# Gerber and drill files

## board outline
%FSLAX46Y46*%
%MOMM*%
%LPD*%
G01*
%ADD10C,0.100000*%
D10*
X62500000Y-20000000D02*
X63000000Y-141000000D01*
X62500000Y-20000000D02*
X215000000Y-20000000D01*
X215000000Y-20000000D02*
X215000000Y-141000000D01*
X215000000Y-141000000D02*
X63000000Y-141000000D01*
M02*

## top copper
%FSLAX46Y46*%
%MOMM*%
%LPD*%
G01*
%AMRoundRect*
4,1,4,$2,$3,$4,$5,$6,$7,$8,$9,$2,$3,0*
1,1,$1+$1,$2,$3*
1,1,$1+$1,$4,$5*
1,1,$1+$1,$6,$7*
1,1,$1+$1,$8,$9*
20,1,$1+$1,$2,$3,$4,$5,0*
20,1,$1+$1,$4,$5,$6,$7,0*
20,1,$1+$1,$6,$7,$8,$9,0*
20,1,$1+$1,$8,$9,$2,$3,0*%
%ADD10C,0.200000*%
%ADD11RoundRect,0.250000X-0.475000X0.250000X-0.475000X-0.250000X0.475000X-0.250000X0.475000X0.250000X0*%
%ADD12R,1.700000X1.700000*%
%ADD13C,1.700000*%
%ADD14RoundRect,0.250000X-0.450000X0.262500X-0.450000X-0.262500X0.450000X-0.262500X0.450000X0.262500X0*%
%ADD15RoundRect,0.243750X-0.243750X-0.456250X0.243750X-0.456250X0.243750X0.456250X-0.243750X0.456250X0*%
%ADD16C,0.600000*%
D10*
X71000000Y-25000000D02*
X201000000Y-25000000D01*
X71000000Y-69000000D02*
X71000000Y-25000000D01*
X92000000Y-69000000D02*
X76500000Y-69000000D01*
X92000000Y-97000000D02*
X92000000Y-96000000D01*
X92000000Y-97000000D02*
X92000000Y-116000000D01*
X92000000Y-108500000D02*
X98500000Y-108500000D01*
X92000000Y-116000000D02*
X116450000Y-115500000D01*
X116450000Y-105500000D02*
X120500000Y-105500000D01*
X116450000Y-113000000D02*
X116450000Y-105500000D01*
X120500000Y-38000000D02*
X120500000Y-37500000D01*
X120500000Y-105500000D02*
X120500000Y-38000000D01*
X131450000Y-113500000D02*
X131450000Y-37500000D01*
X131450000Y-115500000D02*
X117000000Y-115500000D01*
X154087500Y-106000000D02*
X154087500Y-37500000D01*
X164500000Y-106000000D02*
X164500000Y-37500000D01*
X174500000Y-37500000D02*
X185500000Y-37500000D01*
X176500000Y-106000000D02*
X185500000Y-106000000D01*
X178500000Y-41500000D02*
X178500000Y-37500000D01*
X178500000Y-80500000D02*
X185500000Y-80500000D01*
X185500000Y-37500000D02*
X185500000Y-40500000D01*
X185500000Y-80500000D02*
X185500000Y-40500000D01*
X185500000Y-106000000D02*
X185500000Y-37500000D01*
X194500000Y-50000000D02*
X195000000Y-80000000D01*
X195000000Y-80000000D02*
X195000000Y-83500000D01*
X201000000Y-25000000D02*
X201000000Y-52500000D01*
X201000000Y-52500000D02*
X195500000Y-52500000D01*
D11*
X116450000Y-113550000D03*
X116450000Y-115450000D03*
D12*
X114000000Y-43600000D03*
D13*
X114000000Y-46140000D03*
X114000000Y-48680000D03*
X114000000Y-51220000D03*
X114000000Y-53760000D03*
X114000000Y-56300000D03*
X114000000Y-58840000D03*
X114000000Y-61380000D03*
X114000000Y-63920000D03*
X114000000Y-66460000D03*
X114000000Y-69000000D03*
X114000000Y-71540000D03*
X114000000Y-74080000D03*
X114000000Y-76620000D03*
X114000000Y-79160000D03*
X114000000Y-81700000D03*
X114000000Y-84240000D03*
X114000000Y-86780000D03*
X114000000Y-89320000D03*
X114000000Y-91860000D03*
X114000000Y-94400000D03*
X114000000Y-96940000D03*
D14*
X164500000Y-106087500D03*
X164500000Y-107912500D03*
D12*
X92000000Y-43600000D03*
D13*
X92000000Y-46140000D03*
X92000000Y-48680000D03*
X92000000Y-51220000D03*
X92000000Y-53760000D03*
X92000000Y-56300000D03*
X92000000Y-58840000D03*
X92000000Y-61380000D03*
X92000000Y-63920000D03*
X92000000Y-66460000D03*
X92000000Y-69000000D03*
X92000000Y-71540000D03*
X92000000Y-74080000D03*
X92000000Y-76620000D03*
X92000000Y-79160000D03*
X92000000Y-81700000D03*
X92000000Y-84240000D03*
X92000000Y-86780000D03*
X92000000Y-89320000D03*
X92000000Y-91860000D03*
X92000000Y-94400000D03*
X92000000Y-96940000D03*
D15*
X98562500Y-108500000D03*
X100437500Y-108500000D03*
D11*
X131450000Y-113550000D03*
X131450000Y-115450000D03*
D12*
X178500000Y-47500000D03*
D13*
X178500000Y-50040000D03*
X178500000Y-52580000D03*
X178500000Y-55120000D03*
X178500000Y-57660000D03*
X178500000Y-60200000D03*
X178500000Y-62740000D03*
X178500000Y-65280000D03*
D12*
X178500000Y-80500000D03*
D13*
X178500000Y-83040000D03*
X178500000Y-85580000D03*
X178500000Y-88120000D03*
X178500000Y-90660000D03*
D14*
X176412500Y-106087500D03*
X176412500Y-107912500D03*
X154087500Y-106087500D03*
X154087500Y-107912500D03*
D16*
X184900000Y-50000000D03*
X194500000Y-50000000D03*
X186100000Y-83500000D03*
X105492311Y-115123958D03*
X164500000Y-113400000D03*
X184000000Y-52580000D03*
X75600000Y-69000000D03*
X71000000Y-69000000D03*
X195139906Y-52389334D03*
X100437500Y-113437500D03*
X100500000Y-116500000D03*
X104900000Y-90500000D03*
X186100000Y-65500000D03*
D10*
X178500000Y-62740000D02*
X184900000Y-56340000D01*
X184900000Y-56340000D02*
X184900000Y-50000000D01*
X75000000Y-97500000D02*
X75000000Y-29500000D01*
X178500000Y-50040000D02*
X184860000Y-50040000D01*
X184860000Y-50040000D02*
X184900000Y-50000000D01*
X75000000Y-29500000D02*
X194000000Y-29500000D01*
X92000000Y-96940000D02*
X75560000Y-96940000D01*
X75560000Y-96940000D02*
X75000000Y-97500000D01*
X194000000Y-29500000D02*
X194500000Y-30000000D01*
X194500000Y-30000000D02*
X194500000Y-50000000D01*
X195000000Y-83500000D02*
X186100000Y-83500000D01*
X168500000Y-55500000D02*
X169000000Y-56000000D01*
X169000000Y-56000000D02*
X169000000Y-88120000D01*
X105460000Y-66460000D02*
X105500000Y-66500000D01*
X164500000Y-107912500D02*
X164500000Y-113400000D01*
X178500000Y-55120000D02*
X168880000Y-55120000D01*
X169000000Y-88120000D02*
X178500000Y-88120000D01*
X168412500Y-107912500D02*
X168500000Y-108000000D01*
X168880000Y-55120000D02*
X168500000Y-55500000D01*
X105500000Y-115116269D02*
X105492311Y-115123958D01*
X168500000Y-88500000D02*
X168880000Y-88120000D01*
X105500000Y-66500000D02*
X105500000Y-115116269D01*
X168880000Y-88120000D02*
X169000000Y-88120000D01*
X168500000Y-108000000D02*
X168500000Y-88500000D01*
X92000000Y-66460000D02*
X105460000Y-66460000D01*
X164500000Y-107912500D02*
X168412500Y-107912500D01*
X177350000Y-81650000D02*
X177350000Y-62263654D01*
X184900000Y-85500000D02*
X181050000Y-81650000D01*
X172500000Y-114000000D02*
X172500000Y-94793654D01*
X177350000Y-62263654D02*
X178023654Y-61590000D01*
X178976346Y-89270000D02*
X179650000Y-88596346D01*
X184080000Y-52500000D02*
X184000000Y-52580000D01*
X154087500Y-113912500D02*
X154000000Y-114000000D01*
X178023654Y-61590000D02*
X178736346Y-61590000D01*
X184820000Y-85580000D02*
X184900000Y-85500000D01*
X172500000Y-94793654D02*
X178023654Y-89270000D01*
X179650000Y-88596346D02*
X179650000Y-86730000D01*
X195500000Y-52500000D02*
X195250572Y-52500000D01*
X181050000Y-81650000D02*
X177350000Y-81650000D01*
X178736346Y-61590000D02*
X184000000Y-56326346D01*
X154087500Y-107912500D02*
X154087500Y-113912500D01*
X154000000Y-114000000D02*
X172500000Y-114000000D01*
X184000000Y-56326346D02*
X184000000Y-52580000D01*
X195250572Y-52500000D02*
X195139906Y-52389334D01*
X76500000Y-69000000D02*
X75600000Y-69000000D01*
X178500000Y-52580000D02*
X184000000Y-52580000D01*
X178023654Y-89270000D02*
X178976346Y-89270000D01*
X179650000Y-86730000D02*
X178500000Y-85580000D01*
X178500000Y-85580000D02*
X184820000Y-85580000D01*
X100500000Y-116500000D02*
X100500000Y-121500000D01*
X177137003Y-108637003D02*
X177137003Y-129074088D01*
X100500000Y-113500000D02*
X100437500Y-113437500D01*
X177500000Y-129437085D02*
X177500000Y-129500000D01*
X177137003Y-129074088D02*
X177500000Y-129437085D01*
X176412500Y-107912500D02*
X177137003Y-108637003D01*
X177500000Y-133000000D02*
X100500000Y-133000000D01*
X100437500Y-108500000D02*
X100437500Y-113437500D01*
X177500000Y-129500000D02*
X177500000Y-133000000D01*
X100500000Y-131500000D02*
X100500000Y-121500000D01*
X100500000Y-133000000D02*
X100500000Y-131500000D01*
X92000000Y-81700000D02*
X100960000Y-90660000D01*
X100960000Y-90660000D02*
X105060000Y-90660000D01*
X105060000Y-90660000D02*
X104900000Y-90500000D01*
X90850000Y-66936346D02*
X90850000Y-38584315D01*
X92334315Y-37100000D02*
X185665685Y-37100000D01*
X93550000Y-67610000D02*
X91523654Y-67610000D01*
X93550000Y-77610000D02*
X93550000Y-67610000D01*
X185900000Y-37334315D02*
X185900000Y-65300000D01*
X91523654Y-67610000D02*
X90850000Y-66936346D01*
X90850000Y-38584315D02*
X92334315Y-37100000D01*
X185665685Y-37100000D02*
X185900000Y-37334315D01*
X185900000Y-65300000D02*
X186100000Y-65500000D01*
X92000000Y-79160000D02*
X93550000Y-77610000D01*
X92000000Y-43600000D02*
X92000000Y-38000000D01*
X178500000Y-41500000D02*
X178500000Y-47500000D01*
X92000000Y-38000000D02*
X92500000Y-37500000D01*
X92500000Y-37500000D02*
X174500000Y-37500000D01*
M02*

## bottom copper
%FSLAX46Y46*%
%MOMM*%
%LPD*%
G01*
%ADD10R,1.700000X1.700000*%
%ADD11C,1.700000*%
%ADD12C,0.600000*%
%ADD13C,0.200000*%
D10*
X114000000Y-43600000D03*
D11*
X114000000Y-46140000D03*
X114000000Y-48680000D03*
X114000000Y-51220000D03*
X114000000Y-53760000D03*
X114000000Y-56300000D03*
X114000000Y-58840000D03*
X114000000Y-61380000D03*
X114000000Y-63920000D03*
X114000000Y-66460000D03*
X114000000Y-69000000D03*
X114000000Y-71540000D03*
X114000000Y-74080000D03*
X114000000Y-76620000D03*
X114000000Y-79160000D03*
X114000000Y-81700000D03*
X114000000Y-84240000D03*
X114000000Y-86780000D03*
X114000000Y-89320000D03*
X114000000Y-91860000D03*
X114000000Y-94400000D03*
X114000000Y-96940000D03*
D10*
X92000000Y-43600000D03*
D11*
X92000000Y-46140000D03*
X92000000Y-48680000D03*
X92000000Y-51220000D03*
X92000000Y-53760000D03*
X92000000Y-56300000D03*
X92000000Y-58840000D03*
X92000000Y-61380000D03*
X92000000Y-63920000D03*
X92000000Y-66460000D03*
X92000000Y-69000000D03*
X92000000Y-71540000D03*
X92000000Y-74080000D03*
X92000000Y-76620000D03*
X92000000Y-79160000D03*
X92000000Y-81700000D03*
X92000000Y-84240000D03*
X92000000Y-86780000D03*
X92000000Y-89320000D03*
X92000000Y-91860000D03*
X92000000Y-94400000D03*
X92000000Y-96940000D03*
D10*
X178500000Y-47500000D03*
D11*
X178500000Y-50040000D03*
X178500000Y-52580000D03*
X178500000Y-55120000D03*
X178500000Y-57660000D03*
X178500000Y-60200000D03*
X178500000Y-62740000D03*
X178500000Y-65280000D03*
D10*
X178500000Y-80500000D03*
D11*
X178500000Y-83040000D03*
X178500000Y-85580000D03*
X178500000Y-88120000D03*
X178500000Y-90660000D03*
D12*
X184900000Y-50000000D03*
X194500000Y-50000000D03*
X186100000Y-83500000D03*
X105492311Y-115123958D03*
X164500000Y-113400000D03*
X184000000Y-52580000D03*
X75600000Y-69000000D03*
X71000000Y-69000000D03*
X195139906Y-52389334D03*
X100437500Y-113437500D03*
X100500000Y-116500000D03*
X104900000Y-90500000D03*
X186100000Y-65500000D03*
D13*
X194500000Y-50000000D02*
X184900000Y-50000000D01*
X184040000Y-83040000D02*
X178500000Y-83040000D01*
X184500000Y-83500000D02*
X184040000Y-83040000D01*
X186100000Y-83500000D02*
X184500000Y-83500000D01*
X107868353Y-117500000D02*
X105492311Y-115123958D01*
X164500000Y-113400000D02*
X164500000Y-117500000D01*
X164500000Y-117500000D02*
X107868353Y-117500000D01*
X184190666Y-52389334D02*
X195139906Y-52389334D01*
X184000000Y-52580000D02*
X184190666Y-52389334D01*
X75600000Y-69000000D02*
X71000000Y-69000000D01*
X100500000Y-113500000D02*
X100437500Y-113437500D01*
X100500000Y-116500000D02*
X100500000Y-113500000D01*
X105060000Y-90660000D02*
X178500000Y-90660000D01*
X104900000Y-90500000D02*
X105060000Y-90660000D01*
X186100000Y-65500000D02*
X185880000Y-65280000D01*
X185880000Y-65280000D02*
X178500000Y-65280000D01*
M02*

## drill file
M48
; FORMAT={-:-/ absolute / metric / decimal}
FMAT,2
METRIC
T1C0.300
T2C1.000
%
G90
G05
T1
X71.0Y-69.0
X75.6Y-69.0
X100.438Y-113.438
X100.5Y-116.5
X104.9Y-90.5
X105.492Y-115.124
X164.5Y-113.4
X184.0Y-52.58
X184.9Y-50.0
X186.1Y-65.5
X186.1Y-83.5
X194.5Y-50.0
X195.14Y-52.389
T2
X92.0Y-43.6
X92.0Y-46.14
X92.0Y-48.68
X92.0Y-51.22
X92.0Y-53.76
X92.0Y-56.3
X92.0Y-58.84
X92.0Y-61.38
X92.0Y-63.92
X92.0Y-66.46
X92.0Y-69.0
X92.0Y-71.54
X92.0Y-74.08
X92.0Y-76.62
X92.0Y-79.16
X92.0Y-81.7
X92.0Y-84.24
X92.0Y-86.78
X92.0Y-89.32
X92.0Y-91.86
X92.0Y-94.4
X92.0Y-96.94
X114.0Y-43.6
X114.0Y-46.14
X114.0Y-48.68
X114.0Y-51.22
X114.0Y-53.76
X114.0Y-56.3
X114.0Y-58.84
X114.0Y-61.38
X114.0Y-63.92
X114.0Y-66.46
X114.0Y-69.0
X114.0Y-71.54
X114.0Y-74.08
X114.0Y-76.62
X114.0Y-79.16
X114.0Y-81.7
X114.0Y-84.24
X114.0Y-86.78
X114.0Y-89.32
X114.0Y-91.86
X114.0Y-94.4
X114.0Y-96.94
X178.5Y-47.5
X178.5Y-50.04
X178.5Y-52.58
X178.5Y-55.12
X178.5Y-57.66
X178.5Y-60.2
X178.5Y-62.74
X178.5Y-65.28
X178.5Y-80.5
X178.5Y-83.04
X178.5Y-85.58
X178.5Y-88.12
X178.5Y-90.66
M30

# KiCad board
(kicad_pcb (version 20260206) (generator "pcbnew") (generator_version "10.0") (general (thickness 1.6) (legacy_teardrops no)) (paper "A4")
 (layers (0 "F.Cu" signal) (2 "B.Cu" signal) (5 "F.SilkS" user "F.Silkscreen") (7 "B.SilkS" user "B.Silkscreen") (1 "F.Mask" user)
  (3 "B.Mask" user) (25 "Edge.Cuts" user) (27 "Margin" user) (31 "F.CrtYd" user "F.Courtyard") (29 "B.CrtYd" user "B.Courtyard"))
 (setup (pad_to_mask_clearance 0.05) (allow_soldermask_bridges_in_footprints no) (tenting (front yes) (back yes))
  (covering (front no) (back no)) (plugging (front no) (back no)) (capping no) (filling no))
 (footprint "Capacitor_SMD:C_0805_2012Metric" (layer "F.Cu") (at 116.45 114.5 -90)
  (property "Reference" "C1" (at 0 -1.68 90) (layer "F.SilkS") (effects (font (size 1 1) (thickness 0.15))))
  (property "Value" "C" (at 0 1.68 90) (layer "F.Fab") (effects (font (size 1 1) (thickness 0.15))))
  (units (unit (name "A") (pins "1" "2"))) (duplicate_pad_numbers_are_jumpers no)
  (pad "1" smd roundrect (at -0.95 0 270) (size 1 1.45) (layers "F.Cu" "F.Mask" "F.Paste") (roundrect_rratio 0.25) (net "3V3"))
  (pad "2" smd roundrect (at 0.95 0 270) (size 1 1.45) (layers "F.Cu" "F.Mask" "F.Paste") (roundrect_rratio 0.25) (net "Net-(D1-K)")))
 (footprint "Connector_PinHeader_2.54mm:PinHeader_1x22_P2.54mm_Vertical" (layer "F.Cu") (at 114 43.6)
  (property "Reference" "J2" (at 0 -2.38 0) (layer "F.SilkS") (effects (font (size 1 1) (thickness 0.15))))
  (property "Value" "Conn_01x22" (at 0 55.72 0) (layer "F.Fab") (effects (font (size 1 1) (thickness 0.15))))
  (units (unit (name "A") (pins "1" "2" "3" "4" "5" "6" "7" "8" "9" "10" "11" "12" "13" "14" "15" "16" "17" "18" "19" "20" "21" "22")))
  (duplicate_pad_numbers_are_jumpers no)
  (pad "1" thru_hole rect (at 0 0) (size 1.7 1.7) (drill 1) (layers "*.Cu" "*.Mask") (remove_unused_layers no)
   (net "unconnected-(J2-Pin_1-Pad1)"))
  (pad "2" thru_hole circle (at 0 2.54) (size 1.7 1.7) (drill 1) (layers "*.Cu" "*.Mask") (remove_unused_layers no)
   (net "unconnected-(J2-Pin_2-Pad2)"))
  (pad "3" thru_hole circle (at 0 5.08) (size 1.7 1.7) (drill 1) (layers "*.Cu" "*.Mask") (remove_unused_layers no)
   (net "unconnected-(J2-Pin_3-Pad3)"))
  (pad "4" thru_hole circle (at 0 7.62) (size 1.7 1.7) (drill 1) (layers "*.Cu" "*.Mask") (remove_unused_layers no)
   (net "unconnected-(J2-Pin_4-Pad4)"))
  (pad "5" thru_hole circle (at 0 10.16) (size 1.7 1.7) (drill 1) (layers "*.Cu" "*.Mask") (remove_unused_layers no)
   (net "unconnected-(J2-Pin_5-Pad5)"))
  (pad "6" thru_hole circle (at 0 12.7) (size 1.7 1.7) (drill 1) (layers "*.Cu" "*.Mask") (remove_unused_layers no)
   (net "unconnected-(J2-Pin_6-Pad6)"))
  (pad "7" thru_hole circle (at 0 15.24) (size 1.7 1.7) (drill 1) (layers "*.Cu" "*.Mask") (remove_unused_layers no)
   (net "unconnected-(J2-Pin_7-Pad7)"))
  (pad "8" thru_hole circle (at 0 17.78) (size 1.7 1.7) (drill 1) (layers "*.Cu" "*.Mask") (remove_unused_layers no)
   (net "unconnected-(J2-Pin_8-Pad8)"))
  (pad "9" thru_hole circle (at 0 20.32) (size 1.7 1.7) (drill 1) (layers "*.Cu" "*.Mask") (remove_unused_layers no)
   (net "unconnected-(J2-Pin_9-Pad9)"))
  (pad "10" thru_hole circle (at 0 22.86) (size 1.7 1.7) (drill 1) (layers "*.Cu" "*.Mask") (remove_unused_layers no)
   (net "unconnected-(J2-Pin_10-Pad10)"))
  (pad "11" thru_hole circle (at 0 25.4) (size 1.7 1.7) (drill 1) (layers "*.Cu" "*.Mask") (remove_unused_layers no)
   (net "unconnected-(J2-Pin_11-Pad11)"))
  (pad "12" thru_hole circle (at 0 27.94) (size 1.7 1.7) (drill 1) (layers "*.Cu" "*.Mask") (remove_unused_layers no)
   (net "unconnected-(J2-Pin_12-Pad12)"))
  (pad "13" thru_hole circle (at 0 30.48) (size 1.7 1.7) (drill 1) (layers "*.Cu" "*.Mask") (remove_unused_layers no)
   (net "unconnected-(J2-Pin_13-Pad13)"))
  (pad "14" thru_hole circle (at 0 33.02) (size 1.7 1.7) (drill 1) (layers "*.Cu" "*.Mask") (remove_unused_layers no)
   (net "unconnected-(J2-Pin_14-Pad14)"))
  (pad "15" thru_hole circle (at 0 35.56) (size 1.7 1.7) (drill 1) (layers "*.Cu" "*.Mask") (remove_unused_layers no)
   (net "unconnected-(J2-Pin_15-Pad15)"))
  (pad "16" thru_hole circle (at 0 38.1) (size 1.7 1.7) (drill 1) (layers "*.Cu" "*.Mask") (remove_unused_layers no)
   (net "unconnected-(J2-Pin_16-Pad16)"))
  (pad "17" thru_hole circle (at 0 40.64) (size 1.7 1.7) (drill 1) (layers "*.Cu" "*.Mask") (remove_unused_layers no)
   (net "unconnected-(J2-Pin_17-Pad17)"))
  (pad "18" thru_hole circle (at 0 43.18) (size 1.7 1.7) (drill 1) (layers "*.Cu" "*.Mask") (remove_unused_layers no)
   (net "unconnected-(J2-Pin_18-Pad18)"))
  (pad "19" thru_hole circle (at 0 45.72) (size 1.7 1.7) (drill 1) (layers "*.Cu" "*.Mask") (remove_unused_layers no)
   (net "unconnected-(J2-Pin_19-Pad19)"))
  (pad "20" thru_hole circle (at 0 48.26) (size 1.7 1.7) (drill 1) (layers "*.Cu" "*.Mask") (remove_unused_layers no)
   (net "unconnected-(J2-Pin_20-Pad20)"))
  (pad "21" thru_hole circle (at 0 50.8) (size 1.7 1.7) (drill 1) (layers "*.Cu" "*.Mask") (remove_unused_layers no)
   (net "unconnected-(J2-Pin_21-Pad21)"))
  (pad "22" thru_hole circle (at 0 53.34) (size 1.7 1.7) (drill 1) (layers "*.Cu" "*.Mask") (remove_unused_layers no)
   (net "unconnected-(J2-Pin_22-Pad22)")))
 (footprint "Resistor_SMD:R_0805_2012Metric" (layer "F.Cu") (at 164.5 107 -90)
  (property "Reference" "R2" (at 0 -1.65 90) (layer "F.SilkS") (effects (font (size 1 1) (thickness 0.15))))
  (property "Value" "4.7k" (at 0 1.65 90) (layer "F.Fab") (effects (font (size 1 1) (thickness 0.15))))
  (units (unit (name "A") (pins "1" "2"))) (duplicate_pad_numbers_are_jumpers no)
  (pad "1" smd roundrect (at -0.9125 0 270) (size 1.025 1.4) (layers "F.Cu" "F.Mask" "F.Paste") (roundrect_rratio 0.243902) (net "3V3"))
  (pad "2" smd roundrect (at 0.9125 0 270) (size 1.025 1.4) (layers "F.Cu" "F.Mask" "F.Paste") (roundrect_rratio 0.243902)
   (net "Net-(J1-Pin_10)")))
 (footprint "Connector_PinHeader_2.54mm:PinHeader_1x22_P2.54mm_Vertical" (layer "F.Cu") (at 92 43.6)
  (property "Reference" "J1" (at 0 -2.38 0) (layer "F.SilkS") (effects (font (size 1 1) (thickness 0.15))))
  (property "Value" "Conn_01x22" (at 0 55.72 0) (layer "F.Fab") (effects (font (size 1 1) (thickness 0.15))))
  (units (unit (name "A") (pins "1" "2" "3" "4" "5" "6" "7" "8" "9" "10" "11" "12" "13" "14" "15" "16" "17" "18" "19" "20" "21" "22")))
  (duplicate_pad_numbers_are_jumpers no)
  (pad "1" thru_hole rect (at 0 0) (size 1.7 1.7) (drill 1) (layers "*.Cu" "*.Mask") (remove_unused_layers no) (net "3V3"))
  (pad "2" thru_hole circle (at 0 2.54) (size 1.7 1.7) (drill 1) (layers "*.Cu" "*.Mask") (remove_unused_layers no)
   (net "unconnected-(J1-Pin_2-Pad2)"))
  (pad "3" thru_hole circle (at 0 5.08) (size 1.7 1.7) (drill 1) (layers "*.Cu" "*.Mask") (remove_unused_layers no)
   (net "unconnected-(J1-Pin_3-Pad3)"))
  (pad "4" thru_hole circle (at 0 7.62) (size 1.7 1.7) (drill 1) (layers "*.Cu" "*.Mask") (remove_unused_layers no)
   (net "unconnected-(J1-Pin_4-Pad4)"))
  (pad "5" thru_hole circle (at 0 10.16) (size 1.7 1.7) (drill 1) (layers "*.Cu" "*.Mask") (remove_unused_layers no)
   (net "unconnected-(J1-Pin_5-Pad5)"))
  (pad "6" thru_hole circle (at 0 12.7) (size 1.7 1.7) (drill 1) (layers "*.Cu" "*.Mask") (remove_unused_layers no)
   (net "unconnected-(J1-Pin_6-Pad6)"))
  (pad "7" thru_hole circle (at 0 15.24) (size 1.7 1.7) (drill 1) (layers "*.Cu" "*.Mask") (remove_unused_layers no)
   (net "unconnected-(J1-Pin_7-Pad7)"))
  (pad "8" thru_hole circle (at 0 17.78) (size 1.7 1.7) (drill 1) (layers "*.Cu" "*.Mask") (remove_unused_layers no)
   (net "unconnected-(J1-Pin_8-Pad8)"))
  (pad "9" thru_hole circle (at 0 20.32) (size 1.7 1.7) (drill 1) (layers "*.Cu" "*.Mask") (remove_unused_layers no)
   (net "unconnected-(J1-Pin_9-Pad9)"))
  (pad "10" thru_hole circle (at 0 22.86) (size 1.7 1.7) (drill 1) (layers "*.Cu" "*.Mask") (remove_unused_layers no)
   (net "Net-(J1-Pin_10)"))
  (pad "11" thru_hole circle (at 0 25.4) (size 1.7 1.7) (drill 1) (layers "*.Cu" "*.Mask") (remove_unused_layers no) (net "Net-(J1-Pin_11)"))
  (pad "12" thru_hole circle (at 0 27.94) (size 1.7 1.7) (drill 1) (layers "*.Cu" "*.Mask") (remove_unused_layers no)
   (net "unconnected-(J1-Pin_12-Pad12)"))
  (pad "13" thru_hole circle (at 0 30.48) (size 1.7 1.7) (drill 1) (layers "*.Cu" "*.Mask") (remove_unused_layers no)
   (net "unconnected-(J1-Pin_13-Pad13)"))
  (pad "14" thru_hole circle (at 0 33.02) (size 1.7 1.7) (drill 1) (layers "*.Cu" "*.Mask") (remove_unused_layers no)
   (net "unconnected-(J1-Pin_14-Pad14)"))
  (pad "15" thru_hole circle (at 0 35.56) (size 1.7 1.7) (drill 1) (layers "*.Cu" "*.Mask") (remove_unused_layers no) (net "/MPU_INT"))
  (pad "16" thru_hole circle (at 0 38.1) (size 1.7 1.7) (drill 1) (layers "*.Cu" "*.Mask") (remove_unused_layers no) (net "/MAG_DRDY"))
  (pad "17" thru_hole circle (at 0 40.64) (size 1.7 1.7) (drill 1) (layers "*.Cu" "*.Mask") (remove_unused_layers no)
   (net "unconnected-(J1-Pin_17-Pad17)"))
  (pad "18" thru_hole circle (at 0 43.18) (size 1.7 1.7) (drill 1) (layers "*.Cu" "*.Mask") (remove_unused_layers no)
   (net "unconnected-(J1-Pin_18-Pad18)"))
  (pad "19" thru_hole circle (at 0 45.72) (size 1.7 1.7) (drill 1) (layers "*.Cu" "*.Mask") (remove_unused_layers no)
   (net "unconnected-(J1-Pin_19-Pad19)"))
  (pad "20" thru_hole circle (at 0 48.26) (size 1.7 1.7) (drill 1) (layers "*.Cu" "*.Mask") (remove_unused_layers no)
   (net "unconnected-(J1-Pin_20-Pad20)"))
  (pad "21" thru_hole circle (at 0 50.8) (size 1.7 1.7) (drill 1) (layers "*.Cu" "*.Mask") (remove_unused_layers no)
   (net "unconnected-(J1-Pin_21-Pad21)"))
  (pad "22" thru_hole circle (at 0 53.34) (size 1.7 1.7) (drill 1) (layers "*.Cu" "*.Mask") (remove_unused_layers no) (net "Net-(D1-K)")))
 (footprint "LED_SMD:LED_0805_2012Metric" (layer "F.Cu") (at 99.5 108.5)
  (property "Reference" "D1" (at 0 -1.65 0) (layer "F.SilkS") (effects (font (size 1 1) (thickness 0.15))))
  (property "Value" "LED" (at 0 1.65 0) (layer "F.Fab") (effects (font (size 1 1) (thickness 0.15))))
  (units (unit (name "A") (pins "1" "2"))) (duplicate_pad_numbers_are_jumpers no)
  (pad "1" smd roundrect (at -0.9375 0) (size 0.975 1.4) (layers "F.Cu" "F.Mask" "F.Paste") (roundrect_rratio 0.25) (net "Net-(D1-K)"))
  (pad "2" smd roundrect (at 0.9375 0) (size 0.975 1.4) (layers "F.Cu" "F.Mask" "F.Paste") (roundrect_rratio 0.25) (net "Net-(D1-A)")))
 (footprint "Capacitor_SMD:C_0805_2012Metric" (layer "F.Cu") (at 131.45 114.5 -90)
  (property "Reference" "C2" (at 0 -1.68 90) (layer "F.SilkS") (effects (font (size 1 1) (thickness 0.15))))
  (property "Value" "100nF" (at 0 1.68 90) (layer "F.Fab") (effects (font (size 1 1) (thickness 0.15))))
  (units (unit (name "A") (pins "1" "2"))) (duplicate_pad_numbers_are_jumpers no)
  (pad "1" smd roundrect (at -0.95 0 270) (size 1 1.45) (layers "F.Cu" "F.Mask" "F.Paste") (roundrect_rratio 0.25) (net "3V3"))
  (pad "2" smd roundrect (at 0.95 0 270) (size 1 1.45) (layers "F.Cu" "F.Mask" "F.Paste") (roundrect_rratio 0.25) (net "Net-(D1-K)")))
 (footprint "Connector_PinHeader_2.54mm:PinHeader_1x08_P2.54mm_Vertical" (layer "F.Cu") (at 178.5 47.5)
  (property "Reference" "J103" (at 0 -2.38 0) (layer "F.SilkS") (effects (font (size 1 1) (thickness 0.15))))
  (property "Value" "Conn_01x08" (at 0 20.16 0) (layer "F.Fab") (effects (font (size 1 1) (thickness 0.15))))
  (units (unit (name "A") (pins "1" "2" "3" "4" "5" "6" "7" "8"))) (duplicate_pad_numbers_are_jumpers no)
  (pad "1" thru_hole rect (at 0 0) (size 1.7 1.7) (drill 1) (layers "*.Cu" "*.Mask") (remove_unused_layers no) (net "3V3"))
  (pad "2" thru_hole circle (at 0 2.54) (size 1.7 1.7) (drill 1) (layers "*.Cu" "*.Mask") (remove_unused_layers no) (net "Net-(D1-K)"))
  (pad "3" thru_hole circle (at 0 5.08) (size 1.7 1.7) (drill 1) (layers "*.Cu" "*.Mask") (remove_unused_layers no) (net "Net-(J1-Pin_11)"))
  (pad "4" thru_hole circle (at 0 7.62) (size 1.7 1.7) (drill 1) (layers "*.Cu" "*.Mask") (remove_unused_layers no) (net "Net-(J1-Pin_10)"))
  (pad "5" thru_hole circle (at 0 10.16) (size 1.7 1.7) (drill 1) (layers "*.Cu" "*.Mask") (remove_unused_layers no)
   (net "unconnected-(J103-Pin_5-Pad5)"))
  (pad "6" thru_hole circle (at 0 12.7) (size 1.7 1.7) (drill 1) (layers "*.Cu" "*.Mask") (remove_unused_layers no)
   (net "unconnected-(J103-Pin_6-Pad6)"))
  (pad "7" thru_hole circle (at 0 15.24) (size 1.7 1.7) (drill 1) (layers "*.Cu" "*.Mask") (remove_unused_layers no) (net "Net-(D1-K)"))
  (pad "8" thru_hole circle (at 0 17.78) (size 1.7 1.7) (drill 1) (layers "*.Cu" "*.Mask") (remove_unused_layers no) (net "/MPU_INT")))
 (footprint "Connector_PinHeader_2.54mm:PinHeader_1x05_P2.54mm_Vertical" (layer "F.Cu") (at 178.5 80.5)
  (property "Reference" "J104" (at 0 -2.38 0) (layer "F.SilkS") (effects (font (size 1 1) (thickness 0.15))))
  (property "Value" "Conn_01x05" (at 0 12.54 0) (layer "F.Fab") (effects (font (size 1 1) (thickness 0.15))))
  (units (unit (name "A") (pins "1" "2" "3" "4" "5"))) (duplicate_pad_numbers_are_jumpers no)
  (pad "1" thru_hole rect (at 0 0) (size 1.7 1.7) (drill 1) (layers "*.Cu" "*.Mask") (remove_unused_layers no) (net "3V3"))
  (pad "2" thru_hole circle (at 0 2.54) (size 1.7 1.7) (drill 1) (layers "*.Cu" "*.Mask") (remove_unused_layers no) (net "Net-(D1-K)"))
  (pad "3" thru_hole circle (at 0 5.08) (size 1.7 1.7) (drill 1) (layers "*.Cu" "*.Mask") (remove_unused_layers no) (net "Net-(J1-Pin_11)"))
  (pad "4" thru_hole circle (at 0 7.62) (size 1.7 1.7) (drill 1) (layers "*.Cu" "*.Mask") (remove_unused_layers no) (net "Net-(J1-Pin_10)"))
  (pad "5" thru_hole circle (at 0 10.16) (size 1.7 1.7) (drill 1) (layers "*.Cu" "*.Mask") (remove_unused_layers no) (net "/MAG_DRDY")))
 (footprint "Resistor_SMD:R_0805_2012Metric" (layer "F.Cu") (at 176.4125 107 -90)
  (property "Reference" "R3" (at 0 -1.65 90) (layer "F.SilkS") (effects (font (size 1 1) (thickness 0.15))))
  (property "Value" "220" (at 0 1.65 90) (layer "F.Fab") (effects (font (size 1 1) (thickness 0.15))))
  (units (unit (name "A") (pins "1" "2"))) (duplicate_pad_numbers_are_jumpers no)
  (pad "1" smd roundrect (at -0.9125 0 270) (size 1.025 1.4) (layers "F.Cu" "F.Mask" "F.Paste") (roundrect_rratio 0.243902) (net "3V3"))
  (pad "2" smd roundrect (at 0.9125 0 270) (size 1.025 1.4) (layers "F.Cu" "F.Mask" "F.Paste") (roundrect_rratio 0.243902)
   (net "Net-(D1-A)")))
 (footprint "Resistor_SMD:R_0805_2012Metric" (layer "F.Cu") (at 154.0875 107 -90)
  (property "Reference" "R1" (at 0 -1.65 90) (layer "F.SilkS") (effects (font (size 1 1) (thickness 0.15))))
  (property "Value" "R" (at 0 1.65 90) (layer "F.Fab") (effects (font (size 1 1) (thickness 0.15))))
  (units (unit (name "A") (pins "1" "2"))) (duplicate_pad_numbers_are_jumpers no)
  (pad "1" smd roundrect (at -0.9125 0 270) (size 1.025 1.4) (layers "F.Cu" "F.Mask" "F.Paste") (roundrect_rratio 0.243902) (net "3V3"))
  (pad "2" smd roundrect (at 0.9125 0 270) (size 1.025 1.4) (layers "F.Cu" "F.Mask" "F.Paste") (roundrect_rratio 0.243902)
   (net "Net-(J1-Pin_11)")))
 (gr_line (start 71 25) (end 201 25) (stroke (width 0.2) (type default)) (layer "F.Cu") (net "Net-(J1-Pin_11)"))
 (gr_line (start 71 69) (end 71 25) (stroke (width 0.2) (type default)) (layer "F.Cu") (net "Net-(J1-Pin_11)"))
 (gr_line (start 92 69) (end 76.5 69) (stroke (width 0.2) (type default)) (layer "F.Cu") (net "Net-(J1-Pin_11)"))
 (gr_line (start 92 97) (end 92 96) (stroke (width 0.2) (type default)) (layer "F.Cu") (net "Net-(D1-K)"))
 (gr_line (start 92 97) (end 92 116) (stroke (width 0.2) (type default)) (layer "F.Cu") (net "Net-(D1-K)"))
 (gr_line (start 92 108.5) (end 98.5 108.5) (stroke (width 0.2) (type default)) (layer "F.Cu") (net "Net-(D1-K)"))
 (gr_line (start 92 116) (end 116.45 115.5) (stroke (width 0.2) (type default)) (layer "F.Cu") (net "Net-(D1-K)"))
 (gr_line (start 116.45 105.5) (end 120.5 105.5) (stroke (width 0.2) (type default)) (layer "F.Cu") (net "3V3"))
 (gr_line (start 116.45 113) (end 116.45 105.5) (stroke (width 0.2) (type default)) (layer "F.Cu") (net "3V3"))
 (gr_line (start 120.5 38) (end 120.5 37.5) (stroke (width 0.2) (type default)) (layer "F.Cu") (net "3V3"))
 (gr_line (start 120.5 105.5) (end 120.5 38) (stroke (width 0.2) (type default)) (layer "F.Cu") (net "3V3"))
 (gr_line (start 131.45 113.5) (end 131.45 37.5) (stroke (width 0.2) (type default)) (layer "F.Cu") (net "3V3"))
 (gr_line (start 131.45 115.5) (end 117 115.5) (stroke (width 0.2) (type default)) (layer "F.Cu") (net "Net-(D1-K)"))
 (gr_line (start 154.0875 106) (end 154.0875 37.5) (stroke (width 0.2) (type default)) (layer "F.Cu") (net "3V3"))
 (gr_line (start 164.5 106) (end 164.5 37.5) (stroke (width 0.2) (type default)) (layer "F.Cu") (net "3V3"))
 (gr_line (start 174.5 37.5) (end 185.5 37.5) (stroke (width 0.2) (type default)) (layer "F.Cu") (net "3V3"))
 (gr_line (start 176.5 106) (end 185.5 106) (stroke (width 0.2) (type default)) (layer "F.Cu") (net "3V3"))
 (gr_line (start 178.5 41.5) (end 178.5 37.5) (stroke (width 0.2) (type default)) (layer "F.Cu") (net "3V3"))
 (gr_line (start 178.5 80.5) (end 185.5 80.5) (stroke (width 0.2) (type default)) (layer "F.Cu") (net "3V3"))
 (gr_line (start 185.5 37.5) (end 185.5 40.5) (stroke (width 0.2) (type default)) (layer "F.Cu") (net "3V3"))
 (gr_line (start 185.5 80.5) (end 185.5 40.5) (stroke (width 0.2) (type default)) (layer "F.Cu") (net "3V3"))
 (gr_line (start 185.5 106) (end 185.5 37.5) (stroke (width 0.2) (type default)) (layer "F.Cu") (net "3V3"))
 (gr_line (start 194.5 50) (end 195 80) (stroke (width 0.2) (type default)) (layer "F.Cu") (net "Net-(D1-K)"))
 (gr_line (start 195 80) (end 195 83.5) (stroke (width 0.2) (type default)) (layer "F.Cu") (net "Net-(D1-K)"))
 (gr_line (start 201 25) (end 201 52.5) (stroke (width 0.2) (type default)) (layer "F.Cu") (net "Net-(J1-Pin_11)"))
 (gr_line (start 201 52.5) (end 195.5 52.5) (stroke (width 0.2) (type default)) (layer "F.Cu") (net "Net-(J1-Pin_11)"))
 (gr_line (start 62.5 20) (end 63 141) (stroke (width 0.1) (type default)) (layer "Edge.Cuts"))
 (gr_line (start 62.5 20) (end 215 20) (stroke (width 0.1) (type default)) (layer "Edge.Cuts"))
 (gr_line (start 215 20) (end 215 141) (stroke (width 0.1) (type default)) (layer "Edge.Cuts"))
 (gr_line (start 215 141) (end 63 141) (stroke (width 0.1) (type default)) (layer "Edge.Cuts"))
 (segment (start 178.5 62.74) (end 184.9 56.34) (width 0.2) (layer "F.Cu") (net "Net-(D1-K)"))
 (segment (start 184.9 56.34) (end 184.9 50) (width 0.2) (layer "F.Cu") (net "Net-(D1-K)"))
 (segment (start 75 97.5) (end 75 29.5) (width 0.2) (layer "F.Cu") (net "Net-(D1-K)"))
 (segment (start 178.5 50.04) (end 184.86 50.04) (width 0.2) (layer "F.Cu") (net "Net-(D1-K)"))
 (segment (start 184.86 50.04) (end 184.9 50) (width 0.2) (layer "F.Cu") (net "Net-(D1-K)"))
 (segment (start 75 29.5) (end 194 29.5) (width 0.2) (layer "F.Cu") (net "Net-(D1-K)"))
 (segment (start 92 96.94) (end 75.56 96.94) (width 0.2) (layer "F.Cu") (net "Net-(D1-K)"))
 (segment (start 75.56 96.94) (end 75 97.5) (width 0.2) (layer "F.Cu") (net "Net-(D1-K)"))
 (segment (start 194 29.5) (end 194.5 30) (width 0.2) (layer "F.Cu") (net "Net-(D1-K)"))
 (segment (start 194.5 30) (end 194.5 50) (width 0.2) (layer "F.Cu") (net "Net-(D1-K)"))
 (segment (start 195 83.5) (end 186.1 83.5) (width 0.2) (layer "F.Cu") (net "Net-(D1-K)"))
 (via (at 184.9 50) (size 0.6) (drill 0.3) (layers "F.Cu" "B.Cu") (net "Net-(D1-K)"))
 (via (at 194.5 50) (size 0.6) (drill 0.3) (layers "F.Cu" "B.Cu") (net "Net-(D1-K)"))
 (via (at 186.1 83.5) (size 0.6) (drill 0.3) (layers "F.Cu" "B.Cu") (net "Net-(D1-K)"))
 (segment (start 194.5 50) (end 184.9 50) (width 0.2) (layer "B.Cu") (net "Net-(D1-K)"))
 (segment (start 184.04 83.04) (end 178.5 83.04) (width 0.2) (layer "B.Cu") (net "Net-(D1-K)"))
 (segment (start 184.5 83.5) (end 184.04 83.04) (width 0.2) (layer "B.Cu") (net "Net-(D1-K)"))
 (segment (start 186.1 83.5) (end 184.5 83.5) (width 0.2) (layer "B.Cu") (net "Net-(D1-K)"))
 (segment (start 168.5 55.5) (end 169 56) (width 0.2) (layer "F.Cu") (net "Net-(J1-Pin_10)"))
 (segment (start 169 56) (end 169 88.12) (width 0.2) (layer "F.Cu") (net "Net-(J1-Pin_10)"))
 (segment (start 105.46 66.46) (end 105.5 66.5) (width 0.2) (layer "F.Cu") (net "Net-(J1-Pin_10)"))
 (segment (start 164.5 107.9125) (end 164.5 113.4) (width 0.2) (layer "F.Cu") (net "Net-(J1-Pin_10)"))
 (segment (start 178.5 55.12) (end 168.88 55.12) (width 0.2) (layer "F.Cu") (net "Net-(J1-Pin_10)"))
 (segment (start 169 88.12) (end 178.5 88.12) (width 0.2) (layer "F.Cu") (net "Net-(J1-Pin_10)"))
 (segment (start 168.4125 107.9125) (end 168.5 108) (width 0.2) (layer "F.Cu") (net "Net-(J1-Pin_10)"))
 (segment (start 168.88 55.12) (end 168.5 55.5) (width 0.2) (layer "F.Cu") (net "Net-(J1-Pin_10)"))
 (segment (start 105.5 115.116269) (end 105.492311 115.123958) (width 0.2) (layer "F.Cu") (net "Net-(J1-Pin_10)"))
 (segment (start 168.5 88.5) (end 168.88 88.12) (width 0.2) (layer "F.Cu") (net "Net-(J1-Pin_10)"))
 (segment (start 105.5 66.5) (end 105.5 115.116269) (width 0.2) (layer "F.Cu") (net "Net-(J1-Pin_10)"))
 (segment (start 168.88 88.12) (end 169 88.12) (width 0.2) (layer "F.Cu") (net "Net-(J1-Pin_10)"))
 (segment (start 168.5 108) (end 168.5 88.5) (width 0.2) (layer "F.Cu") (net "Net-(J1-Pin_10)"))
 (segment (start 92 66.46) (end 105.46 66.46) (width 0.2) (layer "F.Cu") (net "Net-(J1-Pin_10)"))
 (segment (start 164.5 107.9125) (end 168.4125 107.9125) (width 0.2) (layer "F.Cu") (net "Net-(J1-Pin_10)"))
 (via (at 105.492311 115.123958) (size 0.6) (drill 0.3) (layers "F.Cu" "B.Cu") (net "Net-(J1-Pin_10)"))
 (via (at 164.5 113.4) (size 0.6) (drill 0.3) (layers "F.Cu" "B.Cu") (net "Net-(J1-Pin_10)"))
 (segment (start 107.868353 117.5) (end 105.492311 115.123958) (width 0.2) (layer "B.Cu") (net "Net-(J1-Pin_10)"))
 (segment (start 164.5 113.4) (end 164.5 117.5) (width 0.2) (layer "B.Cu") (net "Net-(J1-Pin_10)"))
 (segment (start 164.5 117.5) (end 107.868353 117.5) (width 0.2) (layer "B.Cu") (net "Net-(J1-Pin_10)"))
 (segment (start 177.35 81.65) (end 177.35 62.263654) (width 0.2) (layer "F.Cu") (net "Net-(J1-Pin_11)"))
 (segment (start 184.9 85.5) (end 181.05 81.65) (width 0.2) (layer "F.Cu") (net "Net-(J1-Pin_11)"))
 (segment (start 172.5 114) (end 172.5 94.793654) (width 0.2) (layer "F.Cu") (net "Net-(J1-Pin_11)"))
 (segment (start 177.35 62.263654) (end 178.023654 61.59) (width 0.2) (layer "F.Cu") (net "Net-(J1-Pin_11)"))
 (segment (start 178.976346 89.27) (end 179.65 88.596346) (width 0.2) (layer "F.Cu") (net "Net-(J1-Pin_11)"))
 (segment (start 184.08 52.5) (end 184 52.58) (width 0.2) (layer "F.Cu") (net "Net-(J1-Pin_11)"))
 (segment (start 154.0875 113.9125) (end 154 114) (width 0.2) (layer "F.Cu") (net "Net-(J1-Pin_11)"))
 (segment (start 178.023654 61.59) (end 178.736346 61.59) (width 0.2) (layer "F.Cu") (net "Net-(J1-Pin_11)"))
 (segment (start 184.82 85.58) (end 184.9 85.5) (width 0.2) (layer "F.Cu") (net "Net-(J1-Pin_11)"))
 (segment (start 172.5 94.793654) (end 178.023654 89.27) (width 0.2) (layer "F.Cu") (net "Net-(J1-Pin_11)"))
 (segment (start 179.65 88.596346) (end 179.65 86.73) (width 0.2) (layer "F.Cu") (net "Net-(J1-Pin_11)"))
 (segment (start 195.5 52.5) (end 195.250572 52.5) (width 0.2) (layer "F.Cu") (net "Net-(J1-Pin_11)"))
 (segment (start 181.05 81.65) (end 177.35 81.65) (width 0.2) (layer "F.Cu") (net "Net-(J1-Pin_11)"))
 (segment (start 178.736346 61.59) (end 184 56.326346) (width 0.2) (layer "F.Cu") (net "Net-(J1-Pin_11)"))
 (segment (start 154.0875 107.9125) (end 154.0875 113.9125) (width 0.2) (layer "F.Cu") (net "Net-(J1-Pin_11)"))
 (segment (start 154 114) (end 172.5 114) (width 0.2) (layer "F.Cu") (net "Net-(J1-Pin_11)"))
 (segment (start 184 56.326346) (end 184 52.58) (width 0.2) (layer "F.Cu") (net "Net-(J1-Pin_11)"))
 (segment (start 195.250572 52.5) (end 195.139906 52.389334) (width 0.2) (layer "F.Cu") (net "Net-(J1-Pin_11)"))
 (segment (start 76.5 69) (end 75.6 69) (width 0.2) (layer "F.Cu") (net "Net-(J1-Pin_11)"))
 (segment (start 178.5 52.58) (end 184 52.58) (width 0.2) (layer "F.Cu") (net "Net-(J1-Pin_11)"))
 (segment (start 178.023654 89.27) (end 178.976346 89.27) (width 0.2) (layer "F.Cu") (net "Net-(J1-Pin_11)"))
 (segment (start 179.65 86.73) (end 178.5 85.58) (width 0.2) (layer "F.Cu") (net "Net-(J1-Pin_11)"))
 (segment (start 178.5 85.58) (end 184.82 85.58) (width 0.2) (layer "F.Cu") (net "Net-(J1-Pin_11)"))
 (via (at 184 52.58) (size 0.6) (drill 0.3) (layers "F.Cu" "B.Cu") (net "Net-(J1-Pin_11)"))
 (via (at 75.6 69) (size 0.6) (drill 0.3) (layers "F.Cu" "B.Cu") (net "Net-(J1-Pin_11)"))
 (via (at 71 69) (size 0.6) (drill 0.3) (layers "F.Cu" "B.Cu") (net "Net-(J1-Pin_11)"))
 (via (at 195.139906 52.389334) (size 0.6) (drill 0.3) (layers "F.Cu" "B.Cu") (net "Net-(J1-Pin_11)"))
 (segment (start 184.190666 52.389334) (end 195.139906 52.389334) (width 0.2) (layer "B.Cu") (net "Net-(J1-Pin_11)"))
 (segment (start 184 52.58) (end 184.190666 52.389334) (width 0.2) (layer "B.Cu") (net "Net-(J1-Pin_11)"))
 (segment (start 75.6 69) (end 71 69) (width 0.2) (layer "B.Cu") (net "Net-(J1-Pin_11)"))
 (segment (start 100.5 116.5) (end 100.5 121.5) (width 0.2) (layer "F.Cu") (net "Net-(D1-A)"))
 (segment (start 177.137003 108.637003) (end 177.137003 129.074088) (width 0.2) (layer "F.Cu") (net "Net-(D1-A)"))
 (segment (start 100.5 113.5) (end 100.4375 113.4375) (width 0.2) (layer "F.Cu") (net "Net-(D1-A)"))
 (segment (start 177.5 129.437085) (end 177.5 129.5) (width 0.2) (layer "F.Cu") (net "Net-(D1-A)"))
 (segment (start 177.137003 129.074088) (end 177.5 129.437085) (width 0.2) (layer "F.Cu") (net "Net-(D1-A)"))
 (segment (start 176.4125 107.9125) (end 177.137003 108.637003) (width 0.2) (layer "F.Cu") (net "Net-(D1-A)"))
 (segment (start 177.5 133) (end 100.5 133) (width 0.2) (layer "F.Cu") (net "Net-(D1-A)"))
 (segment (start 100.4375 108.5) (end 100.4375 113.4375) (width 0.2) (layer "F.Cu") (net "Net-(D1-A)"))
 (segment (start 177.5 129.5) (end 177.5 133) (width 0.2) (layer "F.Cu") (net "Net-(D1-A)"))
 (segment (start 100.5 131.5) (end 100.5 121.5) (width 0.2) (layer "F.Cu") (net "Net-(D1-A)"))
 (segment (start 100.5 133) (end 100.5 131.5) (width 0.2) (layer "F.Cu") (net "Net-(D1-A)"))
 (via (at 100.4375 113.4375) (size 0.6) (drill 0.3) (layers "F.Cu" "B.Cu") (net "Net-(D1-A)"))
 (via (at 100.5 116.5) (size 0.6) (drill 0.3) (layers "F.Cu" "B.Cu") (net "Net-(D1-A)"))
 (segment (start 100.5 113.5) (end 100.4375 113.4375) (width 0.2) (layer "B.Cu") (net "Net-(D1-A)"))
 (segment (start 100.5 116.5) (end 100.5 113.5) (width 0.2) (layer "B.Cu") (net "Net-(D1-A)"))
 (segment (start 92 81.7) (end 100.96 90.66) (width 0.2) (layer "F.Cu") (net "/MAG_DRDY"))
 (segment (start 100.96 90.66) (end 105.06 90.66) (width 0.2) (layer "F.Cu") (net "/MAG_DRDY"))
 (segment (start 105.06 90.66) (end 104.9 90.5) (width 0.2) (layer "F.Cu") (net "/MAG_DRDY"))
 (via (at 104.9 90.5) (size 0.6) (drill 0.3) (layers "F.Cu" "B.Cu") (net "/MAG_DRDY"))
 (segment (start 105.06 90.66) (end 178.5 90.66) (width 0.2) (layer "B.Cu") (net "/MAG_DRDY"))
 (segment (start 104.9 90.5) (end 105.06 90.66) (width 0.2) (layer "B.Cu") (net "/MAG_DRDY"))
 (segment (start 90.85 66.936346) (end 90.85 38.584315) (width 0.2) (layer "F.Cu") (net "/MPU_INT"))
 (segment (start 92.334315 37.1) (end 185.665685 37.1) (width 0.2) (layer "F.Cu") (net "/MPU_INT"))
 (segment (start 93.55 67.61) (end 91.523654 67.61) (width 0.2) (layer "F.Cu") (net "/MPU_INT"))
 (segment (start 93.55 77.61) (end 93.55 67.61) (width 0.2) (layer "F.Cu") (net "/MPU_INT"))
 (segment (start 185.9 37.334315) (end 185.9 65.3) (width 0.2) (layer "F.Cu") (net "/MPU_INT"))
 (segment (start 91.523654 67.61) (end 90.85 66.936346) (width 0.2) (layer "F.Cu") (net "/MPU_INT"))
 (segment (start 90.85 38.584315) (end 92.334315 37.1) (width 0.2) (layer "F.Cu") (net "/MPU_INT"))
 (segment (start 185.665685 37.1) (end 185.9 37.334315) (width 0.2) (layer "F.Cu") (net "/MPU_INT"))
 (segment (start 185.9 65.3) (end 186.1 65.5) (width 0.2) (layer "F.Cu") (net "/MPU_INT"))
 (segment (start 92 79.16) (end 93.55 77.61) (width 0.2) (layer "F.Cu") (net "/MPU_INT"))
 (via (at 186.1 65.5) (size 0.6) (drill 0.3) (layers "F.Cu" "B.Cu") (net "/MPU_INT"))
 (segment (start 186.1 65.5) (end 185.88 65.28) (width 0.2) (layer "B.Cu") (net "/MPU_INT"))
 (segment (start 185.88 65.28) (end 178.5 65.28) (width 0.2) (layer "B.Cu") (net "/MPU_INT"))
 (segment (start 92 43.6) (end 92 38) (width 0.2) (layer "F.Cu") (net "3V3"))
 (segment (start 178.5 41.5) (end 178.5 47.5) (width 0.2) (layer "F.Cu") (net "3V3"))
 (segment (start 92 38) (end 92.5 37.5) (width 0.2) (layer "F.Cu") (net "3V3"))
 (segment (start 92.5 37.5) (end 174.5 37.5) (width 0.2) (layer "F.Cu") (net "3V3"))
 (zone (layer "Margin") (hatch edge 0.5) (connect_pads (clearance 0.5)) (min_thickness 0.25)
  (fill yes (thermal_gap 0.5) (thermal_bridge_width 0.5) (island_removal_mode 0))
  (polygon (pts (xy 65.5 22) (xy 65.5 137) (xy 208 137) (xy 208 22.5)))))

